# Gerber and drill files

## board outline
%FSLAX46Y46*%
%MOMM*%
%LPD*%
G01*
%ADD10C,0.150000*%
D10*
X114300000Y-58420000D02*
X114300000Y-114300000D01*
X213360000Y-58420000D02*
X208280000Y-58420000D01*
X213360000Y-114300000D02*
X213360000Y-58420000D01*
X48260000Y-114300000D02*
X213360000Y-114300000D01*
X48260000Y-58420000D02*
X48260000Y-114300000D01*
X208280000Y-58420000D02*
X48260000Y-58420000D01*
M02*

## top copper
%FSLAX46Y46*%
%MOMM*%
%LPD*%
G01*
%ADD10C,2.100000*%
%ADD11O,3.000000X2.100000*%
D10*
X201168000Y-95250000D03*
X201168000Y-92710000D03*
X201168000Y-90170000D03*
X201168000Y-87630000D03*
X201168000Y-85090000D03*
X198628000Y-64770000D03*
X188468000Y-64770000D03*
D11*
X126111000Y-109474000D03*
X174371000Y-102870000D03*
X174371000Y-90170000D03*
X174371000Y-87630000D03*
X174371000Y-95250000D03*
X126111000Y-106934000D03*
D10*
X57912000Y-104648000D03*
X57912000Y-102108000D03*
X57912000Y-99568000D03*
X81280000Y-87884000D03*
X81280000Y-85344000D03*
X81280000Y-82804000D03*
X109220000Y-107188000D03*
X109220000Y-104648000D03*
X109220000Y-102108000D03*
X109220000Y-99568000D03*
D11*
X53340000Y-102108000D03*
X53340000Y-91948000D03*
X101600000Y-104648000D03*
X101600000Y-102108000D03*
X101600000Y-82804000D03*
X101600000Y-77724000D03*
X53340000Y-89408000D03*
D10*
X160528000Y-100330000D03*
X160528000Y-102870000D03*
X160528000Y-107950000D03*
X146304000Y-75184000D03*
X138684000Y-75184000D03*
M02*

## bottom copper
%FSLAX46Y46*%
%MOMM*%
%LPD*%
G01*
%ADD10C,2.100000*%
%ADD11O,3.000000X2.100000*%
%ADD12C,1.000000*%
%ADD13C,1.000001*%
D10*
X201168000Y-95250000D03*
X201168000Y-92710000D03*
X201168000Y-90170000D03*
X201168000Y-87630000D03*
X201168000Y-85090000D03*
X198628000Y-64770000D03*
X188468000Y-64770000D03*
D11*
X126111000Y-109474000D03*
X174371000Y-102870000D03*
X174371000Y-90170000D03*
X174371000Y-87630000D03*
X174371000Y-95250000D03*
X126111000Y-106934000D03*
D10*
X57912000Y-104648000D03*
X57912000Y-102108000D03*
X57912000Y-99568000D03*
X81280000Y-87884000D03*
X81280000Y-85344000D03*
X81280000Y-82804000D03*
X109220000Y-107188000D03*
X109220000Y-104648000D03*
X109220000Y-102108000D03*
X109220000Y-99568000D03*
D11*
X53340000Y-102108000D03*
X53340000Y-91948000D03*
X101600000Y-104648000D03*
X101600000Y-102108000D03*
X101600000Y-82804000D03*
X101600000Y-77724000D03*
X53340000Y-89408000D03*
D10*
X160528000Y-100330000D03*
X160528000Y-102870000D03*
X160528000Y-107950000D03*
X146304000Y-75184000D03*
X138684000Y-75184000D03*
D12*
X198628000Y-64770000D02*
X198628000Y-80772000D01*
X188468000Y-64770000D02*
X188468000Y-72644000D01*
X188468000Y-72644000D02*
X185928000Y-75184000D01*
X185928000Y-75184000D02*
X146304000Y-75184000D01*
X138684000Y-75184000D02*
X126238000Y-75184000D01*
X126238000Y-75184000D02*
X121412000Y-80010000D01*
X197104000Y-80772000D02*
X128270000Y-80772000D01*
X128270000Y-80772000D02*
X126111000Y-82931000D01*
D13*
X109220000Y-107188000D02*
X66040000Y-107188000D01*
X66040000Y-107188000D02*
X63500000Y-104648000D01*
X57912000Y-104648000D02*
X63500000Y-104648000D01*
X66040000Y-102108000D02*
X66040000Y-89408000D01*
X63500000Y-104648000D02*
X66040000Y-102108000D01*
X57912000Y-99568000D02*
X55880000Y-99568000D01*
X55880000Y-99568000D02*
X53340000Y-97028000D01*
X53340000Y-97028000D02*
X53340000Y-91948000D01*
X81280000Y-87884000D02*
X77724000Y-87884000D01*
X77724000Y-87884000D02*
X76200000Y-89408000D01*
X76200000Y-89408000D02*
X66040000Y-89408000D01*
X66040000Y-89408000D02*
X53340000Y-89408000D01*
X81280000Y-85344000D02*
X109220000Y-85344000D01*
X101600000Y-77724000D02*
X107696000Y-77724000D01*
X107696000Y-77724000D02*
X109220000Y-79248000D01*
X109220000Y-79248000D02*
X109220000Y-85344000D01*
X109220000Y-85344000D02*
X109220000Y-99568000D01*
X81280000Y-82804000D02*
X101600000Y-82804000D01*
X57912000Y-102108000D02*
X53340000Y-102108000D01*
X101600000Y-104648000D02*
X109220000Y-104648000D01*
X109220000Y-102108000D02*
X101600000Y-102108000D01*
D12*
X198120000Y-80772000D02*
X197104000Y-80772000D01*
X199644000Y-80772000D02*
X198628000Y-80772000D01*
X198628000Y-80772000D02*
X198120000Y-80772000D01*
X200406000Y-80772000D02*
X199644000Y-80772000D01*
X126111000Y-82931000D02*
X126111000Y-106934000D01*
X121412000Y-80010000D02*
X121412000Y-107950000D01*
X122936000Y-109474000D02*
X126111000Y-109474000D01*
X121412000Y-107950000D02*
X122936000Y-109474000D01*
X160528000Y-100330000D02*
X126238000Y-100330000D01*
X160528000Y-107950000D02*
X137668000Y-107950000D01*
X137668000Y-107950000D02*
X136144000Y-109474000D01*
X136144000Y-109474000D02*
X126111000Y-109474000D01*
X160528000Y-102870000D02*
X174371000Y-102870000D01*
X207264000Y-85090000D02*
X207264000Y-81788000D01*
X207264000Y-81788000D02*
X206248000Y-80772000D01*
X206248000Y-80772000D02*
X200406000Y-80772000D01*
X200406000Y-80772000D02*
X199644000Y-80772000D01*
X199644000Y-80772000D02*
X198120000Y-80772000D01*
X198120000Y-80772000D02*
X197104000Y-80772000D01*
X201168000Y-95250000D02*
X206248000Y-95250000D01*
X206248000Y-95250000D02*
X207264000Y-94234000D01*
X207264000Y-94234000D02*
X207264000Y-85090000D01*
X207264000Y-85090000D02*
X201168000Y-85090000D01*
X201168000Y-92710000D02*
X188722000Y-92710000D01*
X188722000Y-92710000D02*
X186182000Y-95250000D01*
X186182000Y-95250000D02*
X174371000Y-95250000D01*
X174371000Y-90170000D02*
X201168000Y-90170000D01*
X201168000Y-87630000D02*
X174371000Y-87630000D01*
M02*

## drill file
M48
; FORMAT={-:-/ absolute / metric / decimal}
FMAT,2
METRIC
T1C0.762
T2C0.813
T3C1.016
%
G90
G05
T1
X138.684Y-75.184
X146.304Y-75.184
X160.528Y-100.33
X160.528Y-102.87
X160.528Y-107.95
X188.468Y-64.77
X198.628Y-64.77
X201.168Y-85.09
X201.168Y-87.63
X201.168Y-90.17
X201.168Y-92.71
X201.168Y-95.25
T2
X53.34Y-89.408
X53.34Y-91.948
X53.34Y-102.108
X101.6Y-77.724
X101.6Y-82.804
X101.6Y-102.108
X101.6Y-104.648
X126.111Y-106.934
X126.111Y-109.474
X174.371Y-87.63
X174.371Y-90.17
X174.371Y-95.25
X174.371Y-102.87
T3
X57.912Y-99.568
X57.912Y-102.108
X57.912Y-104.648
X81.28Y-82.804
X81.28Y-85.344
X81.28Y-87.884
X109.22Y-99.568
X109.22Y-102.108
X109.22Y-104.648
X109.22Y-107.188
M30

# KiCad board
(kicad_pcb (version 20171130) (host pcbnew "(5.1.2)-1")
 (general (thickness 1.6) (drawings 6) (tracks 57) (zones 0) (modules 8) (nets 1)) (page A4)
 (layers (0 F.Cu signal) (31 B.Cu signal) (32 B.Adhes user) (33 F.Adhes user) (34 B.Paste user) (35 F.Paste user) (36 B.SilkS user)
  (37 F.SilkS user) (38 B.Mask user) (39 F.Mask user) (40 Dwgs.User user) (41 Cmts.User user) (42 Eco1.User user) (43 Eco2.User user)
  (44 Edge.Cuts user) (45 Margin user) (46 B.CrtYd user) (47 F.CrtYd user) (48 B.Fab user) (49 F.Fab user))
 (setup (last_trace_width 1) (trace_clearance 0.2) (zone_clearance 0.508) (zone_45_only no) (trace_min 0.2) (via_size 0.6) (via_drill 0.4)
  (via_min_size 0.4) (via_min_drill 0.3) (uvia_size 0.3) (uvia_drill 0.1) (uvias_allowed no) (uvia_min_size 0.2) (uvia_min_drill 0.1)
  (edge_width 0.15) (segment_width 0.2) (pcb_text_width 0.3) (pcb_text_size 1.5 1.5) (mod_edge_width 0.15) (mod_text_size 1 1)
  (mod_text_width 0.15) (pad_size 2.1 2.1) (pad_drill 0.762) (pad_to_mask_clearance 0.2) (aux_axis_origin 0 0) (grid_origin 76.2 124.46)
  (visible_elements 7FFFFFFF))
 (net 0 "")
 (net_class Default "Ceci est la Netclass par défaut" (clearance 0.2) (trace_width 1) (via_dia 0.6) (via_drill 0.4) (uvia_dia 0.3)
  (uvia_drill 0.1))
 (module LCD (layer F.Cu) (at 203.708 105.41 90)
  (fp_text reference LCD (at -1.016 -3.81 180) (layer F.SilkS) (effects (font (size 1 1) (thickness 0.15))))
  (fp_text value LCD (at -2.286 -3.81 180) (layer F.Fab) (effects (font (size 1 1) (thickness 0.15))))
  (pad VDD thru_hole circle (at 10.16 -2.54 90) (size 2.1 2.1) (drill 0.762) (layers *.Cu *.Mask F.SilkS))
  (pad VSS thru_hole circle (at 12.7 -2.54 90) (size 2.1 2.1) (drill 0.762) (layers *.Cu *.Mask F.SilkS))
  (pad SDA thru_hole circle (at 15.24 -2.54 90) (size 2.1 2.1) (drill 0.762) (layers *.Cu *.Mask F.SilkS))
  (pad SCL thru_hole circle (at 17.78 -2.54 90) (size 2.1 2.1) (drill 0.762) (layers *.Cu *.Mask F.SilkS))
  (pad RST thru_hole circle (at 20.32 -2.54 90) (size 2.1 2.1) (drill 0.762) (layers *.Cu *.Mask F.SilkS))
  (pad A thru_hole circle (at 40.64 -5.08 90) (size 2.1 2.1) (drill 0.762) (layers *.Cu *.Mask F.SilkS))
  (pad K thru_hole circle (at 40.64 -15.24 90) (size 2.1 2.1) (drill 0.762) (layers *.Cu *.Mask F.SilkS)))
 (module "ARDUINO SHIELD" (layer F.Cu) (at 123.571 68.834 270)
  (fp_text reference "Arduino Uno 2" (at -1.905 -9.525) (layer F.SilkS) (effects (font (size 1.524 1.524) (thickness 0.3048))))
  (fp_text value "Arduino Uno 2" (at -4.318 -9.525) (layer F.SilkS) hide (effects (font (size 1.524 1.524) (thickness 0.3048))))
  (pad GND1 thru_hole oval (at 40.64 -2.54) (size 3 2.1) (drill 0.8128) (layers *.Cu *.Mask F.SilkS))
  (pad 11 thru_hole oval (at 34.036 -50.8) (size 3 2.1) (drill 0.8128) (layers *.Cu *.Mask F.SilkS))
  (pad SDA thru_hole oval (at 21.336 -50.8) (size 3 2.1) (drill 0.8128) (layers *.Cu *.Mask F.SilkS))
  (pad SCL thru_hole oval (at 18.796 -50.8) (size 3 2.1) (drill 0.8128) (layers *.Cu *.Mask F.SilkS))
  (pad GND3 thru_hole oval (at 26.416 -50.8) (size 3 2.1) (drill 0.8128) (layers *.Cu *.Mask F.SilkS))
  (pad 5V thru_hole oval (at 38.1 -2.54) (size 3 2.1) (drill 0.8128) (layers *.Cu *.Mask F.SilkS)))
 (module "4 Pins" (layer F.Cu) (at 62.992 114.808 90)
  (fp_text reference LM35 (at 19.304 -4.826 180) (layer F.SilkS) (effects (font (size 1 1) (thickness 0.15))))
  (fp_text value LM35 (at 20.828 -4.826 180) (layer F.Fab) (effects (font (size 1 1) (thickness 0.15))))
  (pad Vcc thru_hole circle (at 10.16 -5.08 90) (size 2.1 2.1) (drill 1.016) (layers *.Cu *.Mask F.SilkS))
  (pad Vout thru_hole circle (at 12.7 -5.08 90) (size 2.1 2.1) (drill 1.016) (layers *.Cu *.Mask F.SilkS))
  (pad GND thru_hole circle (at 15.24 -5.08 90) (size 2.1 2.1) (drill 1.016) (layers *.Cu *.Mask F.SilkS)))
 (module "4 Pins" (layer F.Cu) (at 86.36 98.044 90)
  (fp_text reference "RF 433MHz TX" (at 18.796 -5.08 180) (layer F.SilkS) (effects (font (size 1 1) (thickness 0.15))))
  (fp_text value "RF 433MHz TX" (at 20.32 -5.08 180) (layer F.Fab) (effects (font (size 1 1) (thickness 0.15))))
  (pad Vcc thru_hole circle (at 10.16 -5.08 90) (size 2.1 2.1) (drill 1.016) (layers *.Cu *.Mask F.SilkS))
  (pad GND thru_hole circle (at 12.7 -5.08 90) (size 2.1 2.1) (drill 1.016) (layers *.Cu *.Mask F.SilkS))
  (pad DATA thru_hole circle (at 15.24 -5.08 90) (size 2.1 2.1) (drill 1.016) (layers *.Cu *.Mask F.SilkS)))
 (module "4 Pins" (layer F.Cu) (at 114.3 117.348 90)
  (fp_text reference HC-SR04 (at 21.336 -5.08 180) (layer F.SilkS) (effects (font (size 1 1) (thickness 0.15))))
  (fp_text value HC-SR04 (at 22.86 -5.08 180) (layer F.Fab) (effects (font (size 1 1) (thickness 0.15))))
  (pad Vcc thru_hole circle (at 10.16 -5.08 90) (size 2.1 2.1) (drill 1.016) (layers *.Cu *.Mask F.SilkS))
  (pad Trig thru_hole circle (at 12.7 -5.08 90) (size 2.1 2.1) (drill 1.016) (layers *.Cu *.Mask F.SilkS))
  (pad Echo thru_hole circle (at 15.24 -5.08 90) (size 2.1 2.1) (drill 1.016) (layers *.Cu *.Mask F.SilkS))
  (pad GND thru_hole circle (at 17.78 -5.08 90) (size 2.1 2.1) (drill 1.016) (layers *.Cu *.Mask F.SilkS)))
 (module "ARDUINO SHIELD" (layer F.Cu) (at 50.8 51.308 270)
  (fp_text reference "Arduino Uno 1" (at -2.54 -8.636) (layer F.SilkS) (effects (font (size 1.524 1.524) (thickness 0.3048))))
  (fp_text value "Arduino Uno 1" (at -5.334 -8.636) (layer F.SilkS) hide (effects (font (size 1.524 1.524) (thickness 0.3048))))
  (pad AD0 thru_hole oval (at 50.8 -2.54) (size 3 2.1) (drill 0.8128) (layers *.Cu *.Mask F.SilkS))
  (pad GND1 thru_hole oval (at 40.64 -2.54) (size 3 2.1) (drill 0.8128) (layers *.Cu *.Mask F.SilkS))
  (pad 4 thru_hole oval (at 53.34 -50.8) (size 3 2.1) (drill 0.8128) (layers *.Cu *.Mask F.SilkS))
  (pad 5 thru_hole oval (at 50.8 -50.8) (size 3 2.1) (drill 0.8128) (layers *.Cu *.Mask F.SilkS))
  (pad 12 thru_hole oval (at 31.496 -50.8) (size 3 2.1) (drill 0.8128) (layers *.Cu *.Mask F.SilkS))
  (pad GND3 thru_hole oval (at 26.416 -50.8) (size 3 2.1) (drill 0.8128) (layers *.Cu *.Mask F.SilkS))
  (pad 5V thru_hole oval (at 38.1 -2.54) (size 3 2.1) (drill 0.8128) (layers *.Cu *.Mask F.SilkS)))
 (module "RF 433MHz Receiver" (layer F.Cu) (at 157.988 97.79 270)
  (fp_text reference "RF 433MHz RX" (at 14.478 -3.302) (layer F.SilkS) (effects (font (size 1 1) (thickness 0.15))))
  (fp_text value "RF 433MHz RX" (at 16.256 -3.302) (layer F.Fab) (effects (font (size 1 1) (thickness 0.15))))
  (pad Vcc thru_hole circle (at 2.54 -2.54 270) (size 2.1 2.1) (drill 0.762) (layers *.Cu *.Mask F.SilkS))
  (pad RXD thru_hole circle (at 5.08 -2.54 270) (size 2.1 2.1) (drill 0.762) (layers *.Cu *.Mask F.SilkS))
  (pad GND thru_hole circle (at 10.16 -2.54 270) (size 2.1 2.1) (drill 0.762) (layers *.Cu *.Mask F.SilkS)))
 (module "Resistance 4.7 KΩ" (layer F.Cu) (at 136.144 77.724)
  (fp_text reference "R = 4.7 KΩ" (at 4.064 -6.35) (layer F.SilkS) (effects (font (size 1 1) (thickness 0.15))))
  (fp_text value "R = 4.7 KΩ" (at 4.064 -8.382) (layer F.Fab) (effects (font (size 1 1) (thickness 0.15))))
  (pad 2 thru_hole circle (at 10.16 -2.54) (size 2.1 2.1) (drill 0.762) (layers *.Cu *.Mask F.SilkS))
  (pad 1 thru_hole circle (at 2.54 -2.54) (size 2.1 2.1) (drill 0.762) (layers *.Cu *.Mask F.SilkS)))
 (gr_line (start 114.3 58.42) (end 114.3 114.3) (angle 90) (layer Edge.Cuts) (width 0.15))
 (gr_line (start 213.36 58.42) (end 208.28 58.42) (angle 90) (layer Edge.Cuts) (width 0.15))
 (gr_line (start 213.36 114.3) (end 213.36 58.42) (angle 90) (layer Edge.Cuts) (width 0.15))
 (gr_line (start 48.26 114.3) (end 213.36 114.3) (angle 90) (layer Edge.Cuts) (width 0.15))
 (gr_line (start 48.26 58.42) (end 48.26 114.3) (angle 90) (layer Edge.Cuts) (width 0.15))
 (gr_line (start 208.28 58.42) (end 48.26 58.42) (angle 90) (layer Edge.Cuts) (width 0.15))
 (segment (start 198.628 64.77) (end 198.628 80.772) (width 1) (layer B.Cu) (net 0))
 (segment (start 188.468 64.77) (end 188.468 72.644) (width 1) (layer B.Cu) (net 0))
 (segment (start 188.468 72.644) (end 185.928 75.184) (width 1) (layer B.Cu) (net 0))
 (segment (start 185.928 75.184) (end 146.304 75.184) (width 1) (layer B.Cu) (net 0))
 (segment (start 138.684 75.184) (end 126.238 75.184) (width 1) (layer B.Cu) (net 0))
 (segment (start 126.238 75.184) (end 121.412 80.01) (width 1) (layer B.Cu) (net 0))
 (segment (start 197.104 80.772) (end 128.27 80.772) (width 1) (layer B.Cu) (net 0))
 (segment (start 128.27 80.772) (end 126.111 82.931) (width 1) (layer B.Cu) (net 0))
 (segment (start 109.22 107.188) (end 66.04 107.188) (width 1.000001) (layer B.Cu) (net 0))
 (segment (start 66.04 107.188) (end 63.5 104.648) (width 1.000001) (layer B.Cu) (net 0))
 (segment (start 57.912 104.648) (end 63.5 104.648) (width 1.000001) (layer B.Cu) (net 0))
 (segment (start 66.04 102.108) (end 66.04 89.408) (width 1.000001) (layer B.Cu) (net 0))
 (segment (start 63.5 104.648) (end 66.04 102.108) (width 1.000001) (layer B.Cu) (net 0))
 (segment (start 57.912 99.568) (end 55.88 99.568) (width 1.000001) (layer B.Cu) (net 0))
 (segment (start 55.88 99.568) (end 53.34 97.028) (width 1.000001) (layer B.Cu) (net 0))
 (segment (start 53.34 97.028) (end 53.34 91.948) (width 1.000001) (layer B.Cu) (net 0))
 (segment (start 81.28 87.884) (end 77.724 87.884) (width 1.000001) (layer B.Cu) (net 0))
 (segment (start 77.724 87.884) (end 76.2 89.408) (width 1.000001) (layer B.Cu) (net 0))
 (segment (start 76.2 89.408) (end 66.04 89.408) (width 1.000001) (layer B.Cu) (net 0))
 (segment (start 66.04 89.408) (end 53.34 89.408) (width 1.000001) (layer B.Cu) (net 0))
 (segment (start 81.28 85.344) (end 109.22 85.344) (width 1.000001) (layer B.Cu) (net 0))
 (segment (start 101.6 77.724) (end 107.696 77.724) (width 1.000001) (layer B.Cu) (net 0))
 (segment (start 107.696 77.724) (end 109.22 79.248) (width 1.000001) (layer B.Cu) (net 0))
 (segment (start 109.22 79.248) (end 109.22 85.344) (width 1.000001) (layer B.Cu) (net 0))
 (segment (start 109.22 85.344) (end 109.22 99.568) (width 1.000001) (layer B.Cu) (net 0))
 (segment (start 81.28 82.804) (end 101.6 82.804) (width 1.000001) (layer B.Cu) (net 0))
 (segment (start 57.912 102.108) (end 53.34 102.108) (width 1.000001) (layer B.Cu) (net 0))
 (segment (start 101.6 104.648) (end 109.22 104.648) (width 1.000001) (layer B.Cu) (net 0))
 (segment (start 109.22 102.108) (end 101.6 102.108) (width 1.000001) (layer B.Cu) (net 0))
 (segment (start 198.12 80.772) (end 197.104 80.772) (width 1) (layer B.Cu) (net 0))
 (segment (start 199.644 80.772) (end 198.628 80.772) (width 1) (layer B.Cu) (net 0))
 (segment (start 198.628 80.772) (end 198.12 80.772) (width 1) (layer B.Cu) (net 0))
 (segment (start 200.406 80.772) (end 199.644 80.772) (width 1) (layer B.Cu) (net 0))
 (segment (start 126.111 82.931) (end 126.111 106.934) (width 1) (layer B.Cu) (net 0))
 (segment (start 121.412 80.01) (end 121.412 107.95) (width 1) (layer B.Cu) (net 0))
 (segment (start 122.936 109.474) (end 126.111 109.474) (width 1) (layer B.Cu) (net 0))
 (segment (start 121.412 107.95) (end 122.936 109.474) (width 1) (layer B.Cu) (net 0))
 (segment (start 160.528 100.33) (end 126.238 100.33) (width 1) (layer B.Cu) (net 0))
 (segment (start 160.528 107.95) (end 137.668 107.95) (width 1) (layer B.Cu) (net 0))
 (segment (start 137.668 107.95) (end 136.144 109.474) (width 1) (layer B.Cu) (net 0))
 (segment (start 136.144 109.474) (end 126.111 109.474) (width 1) (layer B.Cu) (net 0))
 (segment (start 160.528 102.87) (end 174.371 102.87) (width 1) (layer B.Cu) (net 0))
 (segment (start 207.264 85.09) (end 207.264 81.788) (width 1) (layer B.Cu) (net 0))
 (segment (start 207.264 81.788) (end 206.248 80.772) (width 1) (layer B.Cu) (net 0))
 (segment (start 206.248 80.772) (end 200.406 80.772) (width 1) (layer B.Cu) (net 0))
 (segment (start 200.406 80.772) (end 199.644 80.772) (width 1) (layer B.Cu) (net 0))
 (segment (start 199.644 80.772) (end 198.12 80.772) (width 1) (layer B.Cu) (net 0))
 (segment (start 198.12 80.772) (end 197.104 80.772) (width 1) (layer B.Cu) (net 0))
 (segment (start 201.168 95.25) (end 206.248 95.25) (width 1) (layer B.Cu) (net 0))
 (segment (start 206.248 95.25) (end 207.264 94.234) (width 1) (layer B.Cu) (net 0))
 (segment (start 207.264 94.234) (end 207.264 85.09) (width 1) (layer B.Cu) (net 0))
 (segment (start 207.264 85.09) (end 201.168 85.09) (width 1) (layer B.Cu) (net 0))
 (segment (start 201.168 92.71) (end 188.722 92.71) (width 1) (layer B.Cu) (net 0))
 (segment (start 188.722 92.71) (end 186.182 95.25) (width 1) (layer B.Cu) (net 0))
 (segment (start 186.182 95.25) (end 174.371 95.25) (width 1) (layer B.Cu) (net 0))
 (segment (start 174.371 90.17) (end 201.168 90.17) (width 1) (layer B.Cu) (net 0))
 (segment (start 201.168 87.63) (end 174.371 87.63) (width 1) (layer B.Cu) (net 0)))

